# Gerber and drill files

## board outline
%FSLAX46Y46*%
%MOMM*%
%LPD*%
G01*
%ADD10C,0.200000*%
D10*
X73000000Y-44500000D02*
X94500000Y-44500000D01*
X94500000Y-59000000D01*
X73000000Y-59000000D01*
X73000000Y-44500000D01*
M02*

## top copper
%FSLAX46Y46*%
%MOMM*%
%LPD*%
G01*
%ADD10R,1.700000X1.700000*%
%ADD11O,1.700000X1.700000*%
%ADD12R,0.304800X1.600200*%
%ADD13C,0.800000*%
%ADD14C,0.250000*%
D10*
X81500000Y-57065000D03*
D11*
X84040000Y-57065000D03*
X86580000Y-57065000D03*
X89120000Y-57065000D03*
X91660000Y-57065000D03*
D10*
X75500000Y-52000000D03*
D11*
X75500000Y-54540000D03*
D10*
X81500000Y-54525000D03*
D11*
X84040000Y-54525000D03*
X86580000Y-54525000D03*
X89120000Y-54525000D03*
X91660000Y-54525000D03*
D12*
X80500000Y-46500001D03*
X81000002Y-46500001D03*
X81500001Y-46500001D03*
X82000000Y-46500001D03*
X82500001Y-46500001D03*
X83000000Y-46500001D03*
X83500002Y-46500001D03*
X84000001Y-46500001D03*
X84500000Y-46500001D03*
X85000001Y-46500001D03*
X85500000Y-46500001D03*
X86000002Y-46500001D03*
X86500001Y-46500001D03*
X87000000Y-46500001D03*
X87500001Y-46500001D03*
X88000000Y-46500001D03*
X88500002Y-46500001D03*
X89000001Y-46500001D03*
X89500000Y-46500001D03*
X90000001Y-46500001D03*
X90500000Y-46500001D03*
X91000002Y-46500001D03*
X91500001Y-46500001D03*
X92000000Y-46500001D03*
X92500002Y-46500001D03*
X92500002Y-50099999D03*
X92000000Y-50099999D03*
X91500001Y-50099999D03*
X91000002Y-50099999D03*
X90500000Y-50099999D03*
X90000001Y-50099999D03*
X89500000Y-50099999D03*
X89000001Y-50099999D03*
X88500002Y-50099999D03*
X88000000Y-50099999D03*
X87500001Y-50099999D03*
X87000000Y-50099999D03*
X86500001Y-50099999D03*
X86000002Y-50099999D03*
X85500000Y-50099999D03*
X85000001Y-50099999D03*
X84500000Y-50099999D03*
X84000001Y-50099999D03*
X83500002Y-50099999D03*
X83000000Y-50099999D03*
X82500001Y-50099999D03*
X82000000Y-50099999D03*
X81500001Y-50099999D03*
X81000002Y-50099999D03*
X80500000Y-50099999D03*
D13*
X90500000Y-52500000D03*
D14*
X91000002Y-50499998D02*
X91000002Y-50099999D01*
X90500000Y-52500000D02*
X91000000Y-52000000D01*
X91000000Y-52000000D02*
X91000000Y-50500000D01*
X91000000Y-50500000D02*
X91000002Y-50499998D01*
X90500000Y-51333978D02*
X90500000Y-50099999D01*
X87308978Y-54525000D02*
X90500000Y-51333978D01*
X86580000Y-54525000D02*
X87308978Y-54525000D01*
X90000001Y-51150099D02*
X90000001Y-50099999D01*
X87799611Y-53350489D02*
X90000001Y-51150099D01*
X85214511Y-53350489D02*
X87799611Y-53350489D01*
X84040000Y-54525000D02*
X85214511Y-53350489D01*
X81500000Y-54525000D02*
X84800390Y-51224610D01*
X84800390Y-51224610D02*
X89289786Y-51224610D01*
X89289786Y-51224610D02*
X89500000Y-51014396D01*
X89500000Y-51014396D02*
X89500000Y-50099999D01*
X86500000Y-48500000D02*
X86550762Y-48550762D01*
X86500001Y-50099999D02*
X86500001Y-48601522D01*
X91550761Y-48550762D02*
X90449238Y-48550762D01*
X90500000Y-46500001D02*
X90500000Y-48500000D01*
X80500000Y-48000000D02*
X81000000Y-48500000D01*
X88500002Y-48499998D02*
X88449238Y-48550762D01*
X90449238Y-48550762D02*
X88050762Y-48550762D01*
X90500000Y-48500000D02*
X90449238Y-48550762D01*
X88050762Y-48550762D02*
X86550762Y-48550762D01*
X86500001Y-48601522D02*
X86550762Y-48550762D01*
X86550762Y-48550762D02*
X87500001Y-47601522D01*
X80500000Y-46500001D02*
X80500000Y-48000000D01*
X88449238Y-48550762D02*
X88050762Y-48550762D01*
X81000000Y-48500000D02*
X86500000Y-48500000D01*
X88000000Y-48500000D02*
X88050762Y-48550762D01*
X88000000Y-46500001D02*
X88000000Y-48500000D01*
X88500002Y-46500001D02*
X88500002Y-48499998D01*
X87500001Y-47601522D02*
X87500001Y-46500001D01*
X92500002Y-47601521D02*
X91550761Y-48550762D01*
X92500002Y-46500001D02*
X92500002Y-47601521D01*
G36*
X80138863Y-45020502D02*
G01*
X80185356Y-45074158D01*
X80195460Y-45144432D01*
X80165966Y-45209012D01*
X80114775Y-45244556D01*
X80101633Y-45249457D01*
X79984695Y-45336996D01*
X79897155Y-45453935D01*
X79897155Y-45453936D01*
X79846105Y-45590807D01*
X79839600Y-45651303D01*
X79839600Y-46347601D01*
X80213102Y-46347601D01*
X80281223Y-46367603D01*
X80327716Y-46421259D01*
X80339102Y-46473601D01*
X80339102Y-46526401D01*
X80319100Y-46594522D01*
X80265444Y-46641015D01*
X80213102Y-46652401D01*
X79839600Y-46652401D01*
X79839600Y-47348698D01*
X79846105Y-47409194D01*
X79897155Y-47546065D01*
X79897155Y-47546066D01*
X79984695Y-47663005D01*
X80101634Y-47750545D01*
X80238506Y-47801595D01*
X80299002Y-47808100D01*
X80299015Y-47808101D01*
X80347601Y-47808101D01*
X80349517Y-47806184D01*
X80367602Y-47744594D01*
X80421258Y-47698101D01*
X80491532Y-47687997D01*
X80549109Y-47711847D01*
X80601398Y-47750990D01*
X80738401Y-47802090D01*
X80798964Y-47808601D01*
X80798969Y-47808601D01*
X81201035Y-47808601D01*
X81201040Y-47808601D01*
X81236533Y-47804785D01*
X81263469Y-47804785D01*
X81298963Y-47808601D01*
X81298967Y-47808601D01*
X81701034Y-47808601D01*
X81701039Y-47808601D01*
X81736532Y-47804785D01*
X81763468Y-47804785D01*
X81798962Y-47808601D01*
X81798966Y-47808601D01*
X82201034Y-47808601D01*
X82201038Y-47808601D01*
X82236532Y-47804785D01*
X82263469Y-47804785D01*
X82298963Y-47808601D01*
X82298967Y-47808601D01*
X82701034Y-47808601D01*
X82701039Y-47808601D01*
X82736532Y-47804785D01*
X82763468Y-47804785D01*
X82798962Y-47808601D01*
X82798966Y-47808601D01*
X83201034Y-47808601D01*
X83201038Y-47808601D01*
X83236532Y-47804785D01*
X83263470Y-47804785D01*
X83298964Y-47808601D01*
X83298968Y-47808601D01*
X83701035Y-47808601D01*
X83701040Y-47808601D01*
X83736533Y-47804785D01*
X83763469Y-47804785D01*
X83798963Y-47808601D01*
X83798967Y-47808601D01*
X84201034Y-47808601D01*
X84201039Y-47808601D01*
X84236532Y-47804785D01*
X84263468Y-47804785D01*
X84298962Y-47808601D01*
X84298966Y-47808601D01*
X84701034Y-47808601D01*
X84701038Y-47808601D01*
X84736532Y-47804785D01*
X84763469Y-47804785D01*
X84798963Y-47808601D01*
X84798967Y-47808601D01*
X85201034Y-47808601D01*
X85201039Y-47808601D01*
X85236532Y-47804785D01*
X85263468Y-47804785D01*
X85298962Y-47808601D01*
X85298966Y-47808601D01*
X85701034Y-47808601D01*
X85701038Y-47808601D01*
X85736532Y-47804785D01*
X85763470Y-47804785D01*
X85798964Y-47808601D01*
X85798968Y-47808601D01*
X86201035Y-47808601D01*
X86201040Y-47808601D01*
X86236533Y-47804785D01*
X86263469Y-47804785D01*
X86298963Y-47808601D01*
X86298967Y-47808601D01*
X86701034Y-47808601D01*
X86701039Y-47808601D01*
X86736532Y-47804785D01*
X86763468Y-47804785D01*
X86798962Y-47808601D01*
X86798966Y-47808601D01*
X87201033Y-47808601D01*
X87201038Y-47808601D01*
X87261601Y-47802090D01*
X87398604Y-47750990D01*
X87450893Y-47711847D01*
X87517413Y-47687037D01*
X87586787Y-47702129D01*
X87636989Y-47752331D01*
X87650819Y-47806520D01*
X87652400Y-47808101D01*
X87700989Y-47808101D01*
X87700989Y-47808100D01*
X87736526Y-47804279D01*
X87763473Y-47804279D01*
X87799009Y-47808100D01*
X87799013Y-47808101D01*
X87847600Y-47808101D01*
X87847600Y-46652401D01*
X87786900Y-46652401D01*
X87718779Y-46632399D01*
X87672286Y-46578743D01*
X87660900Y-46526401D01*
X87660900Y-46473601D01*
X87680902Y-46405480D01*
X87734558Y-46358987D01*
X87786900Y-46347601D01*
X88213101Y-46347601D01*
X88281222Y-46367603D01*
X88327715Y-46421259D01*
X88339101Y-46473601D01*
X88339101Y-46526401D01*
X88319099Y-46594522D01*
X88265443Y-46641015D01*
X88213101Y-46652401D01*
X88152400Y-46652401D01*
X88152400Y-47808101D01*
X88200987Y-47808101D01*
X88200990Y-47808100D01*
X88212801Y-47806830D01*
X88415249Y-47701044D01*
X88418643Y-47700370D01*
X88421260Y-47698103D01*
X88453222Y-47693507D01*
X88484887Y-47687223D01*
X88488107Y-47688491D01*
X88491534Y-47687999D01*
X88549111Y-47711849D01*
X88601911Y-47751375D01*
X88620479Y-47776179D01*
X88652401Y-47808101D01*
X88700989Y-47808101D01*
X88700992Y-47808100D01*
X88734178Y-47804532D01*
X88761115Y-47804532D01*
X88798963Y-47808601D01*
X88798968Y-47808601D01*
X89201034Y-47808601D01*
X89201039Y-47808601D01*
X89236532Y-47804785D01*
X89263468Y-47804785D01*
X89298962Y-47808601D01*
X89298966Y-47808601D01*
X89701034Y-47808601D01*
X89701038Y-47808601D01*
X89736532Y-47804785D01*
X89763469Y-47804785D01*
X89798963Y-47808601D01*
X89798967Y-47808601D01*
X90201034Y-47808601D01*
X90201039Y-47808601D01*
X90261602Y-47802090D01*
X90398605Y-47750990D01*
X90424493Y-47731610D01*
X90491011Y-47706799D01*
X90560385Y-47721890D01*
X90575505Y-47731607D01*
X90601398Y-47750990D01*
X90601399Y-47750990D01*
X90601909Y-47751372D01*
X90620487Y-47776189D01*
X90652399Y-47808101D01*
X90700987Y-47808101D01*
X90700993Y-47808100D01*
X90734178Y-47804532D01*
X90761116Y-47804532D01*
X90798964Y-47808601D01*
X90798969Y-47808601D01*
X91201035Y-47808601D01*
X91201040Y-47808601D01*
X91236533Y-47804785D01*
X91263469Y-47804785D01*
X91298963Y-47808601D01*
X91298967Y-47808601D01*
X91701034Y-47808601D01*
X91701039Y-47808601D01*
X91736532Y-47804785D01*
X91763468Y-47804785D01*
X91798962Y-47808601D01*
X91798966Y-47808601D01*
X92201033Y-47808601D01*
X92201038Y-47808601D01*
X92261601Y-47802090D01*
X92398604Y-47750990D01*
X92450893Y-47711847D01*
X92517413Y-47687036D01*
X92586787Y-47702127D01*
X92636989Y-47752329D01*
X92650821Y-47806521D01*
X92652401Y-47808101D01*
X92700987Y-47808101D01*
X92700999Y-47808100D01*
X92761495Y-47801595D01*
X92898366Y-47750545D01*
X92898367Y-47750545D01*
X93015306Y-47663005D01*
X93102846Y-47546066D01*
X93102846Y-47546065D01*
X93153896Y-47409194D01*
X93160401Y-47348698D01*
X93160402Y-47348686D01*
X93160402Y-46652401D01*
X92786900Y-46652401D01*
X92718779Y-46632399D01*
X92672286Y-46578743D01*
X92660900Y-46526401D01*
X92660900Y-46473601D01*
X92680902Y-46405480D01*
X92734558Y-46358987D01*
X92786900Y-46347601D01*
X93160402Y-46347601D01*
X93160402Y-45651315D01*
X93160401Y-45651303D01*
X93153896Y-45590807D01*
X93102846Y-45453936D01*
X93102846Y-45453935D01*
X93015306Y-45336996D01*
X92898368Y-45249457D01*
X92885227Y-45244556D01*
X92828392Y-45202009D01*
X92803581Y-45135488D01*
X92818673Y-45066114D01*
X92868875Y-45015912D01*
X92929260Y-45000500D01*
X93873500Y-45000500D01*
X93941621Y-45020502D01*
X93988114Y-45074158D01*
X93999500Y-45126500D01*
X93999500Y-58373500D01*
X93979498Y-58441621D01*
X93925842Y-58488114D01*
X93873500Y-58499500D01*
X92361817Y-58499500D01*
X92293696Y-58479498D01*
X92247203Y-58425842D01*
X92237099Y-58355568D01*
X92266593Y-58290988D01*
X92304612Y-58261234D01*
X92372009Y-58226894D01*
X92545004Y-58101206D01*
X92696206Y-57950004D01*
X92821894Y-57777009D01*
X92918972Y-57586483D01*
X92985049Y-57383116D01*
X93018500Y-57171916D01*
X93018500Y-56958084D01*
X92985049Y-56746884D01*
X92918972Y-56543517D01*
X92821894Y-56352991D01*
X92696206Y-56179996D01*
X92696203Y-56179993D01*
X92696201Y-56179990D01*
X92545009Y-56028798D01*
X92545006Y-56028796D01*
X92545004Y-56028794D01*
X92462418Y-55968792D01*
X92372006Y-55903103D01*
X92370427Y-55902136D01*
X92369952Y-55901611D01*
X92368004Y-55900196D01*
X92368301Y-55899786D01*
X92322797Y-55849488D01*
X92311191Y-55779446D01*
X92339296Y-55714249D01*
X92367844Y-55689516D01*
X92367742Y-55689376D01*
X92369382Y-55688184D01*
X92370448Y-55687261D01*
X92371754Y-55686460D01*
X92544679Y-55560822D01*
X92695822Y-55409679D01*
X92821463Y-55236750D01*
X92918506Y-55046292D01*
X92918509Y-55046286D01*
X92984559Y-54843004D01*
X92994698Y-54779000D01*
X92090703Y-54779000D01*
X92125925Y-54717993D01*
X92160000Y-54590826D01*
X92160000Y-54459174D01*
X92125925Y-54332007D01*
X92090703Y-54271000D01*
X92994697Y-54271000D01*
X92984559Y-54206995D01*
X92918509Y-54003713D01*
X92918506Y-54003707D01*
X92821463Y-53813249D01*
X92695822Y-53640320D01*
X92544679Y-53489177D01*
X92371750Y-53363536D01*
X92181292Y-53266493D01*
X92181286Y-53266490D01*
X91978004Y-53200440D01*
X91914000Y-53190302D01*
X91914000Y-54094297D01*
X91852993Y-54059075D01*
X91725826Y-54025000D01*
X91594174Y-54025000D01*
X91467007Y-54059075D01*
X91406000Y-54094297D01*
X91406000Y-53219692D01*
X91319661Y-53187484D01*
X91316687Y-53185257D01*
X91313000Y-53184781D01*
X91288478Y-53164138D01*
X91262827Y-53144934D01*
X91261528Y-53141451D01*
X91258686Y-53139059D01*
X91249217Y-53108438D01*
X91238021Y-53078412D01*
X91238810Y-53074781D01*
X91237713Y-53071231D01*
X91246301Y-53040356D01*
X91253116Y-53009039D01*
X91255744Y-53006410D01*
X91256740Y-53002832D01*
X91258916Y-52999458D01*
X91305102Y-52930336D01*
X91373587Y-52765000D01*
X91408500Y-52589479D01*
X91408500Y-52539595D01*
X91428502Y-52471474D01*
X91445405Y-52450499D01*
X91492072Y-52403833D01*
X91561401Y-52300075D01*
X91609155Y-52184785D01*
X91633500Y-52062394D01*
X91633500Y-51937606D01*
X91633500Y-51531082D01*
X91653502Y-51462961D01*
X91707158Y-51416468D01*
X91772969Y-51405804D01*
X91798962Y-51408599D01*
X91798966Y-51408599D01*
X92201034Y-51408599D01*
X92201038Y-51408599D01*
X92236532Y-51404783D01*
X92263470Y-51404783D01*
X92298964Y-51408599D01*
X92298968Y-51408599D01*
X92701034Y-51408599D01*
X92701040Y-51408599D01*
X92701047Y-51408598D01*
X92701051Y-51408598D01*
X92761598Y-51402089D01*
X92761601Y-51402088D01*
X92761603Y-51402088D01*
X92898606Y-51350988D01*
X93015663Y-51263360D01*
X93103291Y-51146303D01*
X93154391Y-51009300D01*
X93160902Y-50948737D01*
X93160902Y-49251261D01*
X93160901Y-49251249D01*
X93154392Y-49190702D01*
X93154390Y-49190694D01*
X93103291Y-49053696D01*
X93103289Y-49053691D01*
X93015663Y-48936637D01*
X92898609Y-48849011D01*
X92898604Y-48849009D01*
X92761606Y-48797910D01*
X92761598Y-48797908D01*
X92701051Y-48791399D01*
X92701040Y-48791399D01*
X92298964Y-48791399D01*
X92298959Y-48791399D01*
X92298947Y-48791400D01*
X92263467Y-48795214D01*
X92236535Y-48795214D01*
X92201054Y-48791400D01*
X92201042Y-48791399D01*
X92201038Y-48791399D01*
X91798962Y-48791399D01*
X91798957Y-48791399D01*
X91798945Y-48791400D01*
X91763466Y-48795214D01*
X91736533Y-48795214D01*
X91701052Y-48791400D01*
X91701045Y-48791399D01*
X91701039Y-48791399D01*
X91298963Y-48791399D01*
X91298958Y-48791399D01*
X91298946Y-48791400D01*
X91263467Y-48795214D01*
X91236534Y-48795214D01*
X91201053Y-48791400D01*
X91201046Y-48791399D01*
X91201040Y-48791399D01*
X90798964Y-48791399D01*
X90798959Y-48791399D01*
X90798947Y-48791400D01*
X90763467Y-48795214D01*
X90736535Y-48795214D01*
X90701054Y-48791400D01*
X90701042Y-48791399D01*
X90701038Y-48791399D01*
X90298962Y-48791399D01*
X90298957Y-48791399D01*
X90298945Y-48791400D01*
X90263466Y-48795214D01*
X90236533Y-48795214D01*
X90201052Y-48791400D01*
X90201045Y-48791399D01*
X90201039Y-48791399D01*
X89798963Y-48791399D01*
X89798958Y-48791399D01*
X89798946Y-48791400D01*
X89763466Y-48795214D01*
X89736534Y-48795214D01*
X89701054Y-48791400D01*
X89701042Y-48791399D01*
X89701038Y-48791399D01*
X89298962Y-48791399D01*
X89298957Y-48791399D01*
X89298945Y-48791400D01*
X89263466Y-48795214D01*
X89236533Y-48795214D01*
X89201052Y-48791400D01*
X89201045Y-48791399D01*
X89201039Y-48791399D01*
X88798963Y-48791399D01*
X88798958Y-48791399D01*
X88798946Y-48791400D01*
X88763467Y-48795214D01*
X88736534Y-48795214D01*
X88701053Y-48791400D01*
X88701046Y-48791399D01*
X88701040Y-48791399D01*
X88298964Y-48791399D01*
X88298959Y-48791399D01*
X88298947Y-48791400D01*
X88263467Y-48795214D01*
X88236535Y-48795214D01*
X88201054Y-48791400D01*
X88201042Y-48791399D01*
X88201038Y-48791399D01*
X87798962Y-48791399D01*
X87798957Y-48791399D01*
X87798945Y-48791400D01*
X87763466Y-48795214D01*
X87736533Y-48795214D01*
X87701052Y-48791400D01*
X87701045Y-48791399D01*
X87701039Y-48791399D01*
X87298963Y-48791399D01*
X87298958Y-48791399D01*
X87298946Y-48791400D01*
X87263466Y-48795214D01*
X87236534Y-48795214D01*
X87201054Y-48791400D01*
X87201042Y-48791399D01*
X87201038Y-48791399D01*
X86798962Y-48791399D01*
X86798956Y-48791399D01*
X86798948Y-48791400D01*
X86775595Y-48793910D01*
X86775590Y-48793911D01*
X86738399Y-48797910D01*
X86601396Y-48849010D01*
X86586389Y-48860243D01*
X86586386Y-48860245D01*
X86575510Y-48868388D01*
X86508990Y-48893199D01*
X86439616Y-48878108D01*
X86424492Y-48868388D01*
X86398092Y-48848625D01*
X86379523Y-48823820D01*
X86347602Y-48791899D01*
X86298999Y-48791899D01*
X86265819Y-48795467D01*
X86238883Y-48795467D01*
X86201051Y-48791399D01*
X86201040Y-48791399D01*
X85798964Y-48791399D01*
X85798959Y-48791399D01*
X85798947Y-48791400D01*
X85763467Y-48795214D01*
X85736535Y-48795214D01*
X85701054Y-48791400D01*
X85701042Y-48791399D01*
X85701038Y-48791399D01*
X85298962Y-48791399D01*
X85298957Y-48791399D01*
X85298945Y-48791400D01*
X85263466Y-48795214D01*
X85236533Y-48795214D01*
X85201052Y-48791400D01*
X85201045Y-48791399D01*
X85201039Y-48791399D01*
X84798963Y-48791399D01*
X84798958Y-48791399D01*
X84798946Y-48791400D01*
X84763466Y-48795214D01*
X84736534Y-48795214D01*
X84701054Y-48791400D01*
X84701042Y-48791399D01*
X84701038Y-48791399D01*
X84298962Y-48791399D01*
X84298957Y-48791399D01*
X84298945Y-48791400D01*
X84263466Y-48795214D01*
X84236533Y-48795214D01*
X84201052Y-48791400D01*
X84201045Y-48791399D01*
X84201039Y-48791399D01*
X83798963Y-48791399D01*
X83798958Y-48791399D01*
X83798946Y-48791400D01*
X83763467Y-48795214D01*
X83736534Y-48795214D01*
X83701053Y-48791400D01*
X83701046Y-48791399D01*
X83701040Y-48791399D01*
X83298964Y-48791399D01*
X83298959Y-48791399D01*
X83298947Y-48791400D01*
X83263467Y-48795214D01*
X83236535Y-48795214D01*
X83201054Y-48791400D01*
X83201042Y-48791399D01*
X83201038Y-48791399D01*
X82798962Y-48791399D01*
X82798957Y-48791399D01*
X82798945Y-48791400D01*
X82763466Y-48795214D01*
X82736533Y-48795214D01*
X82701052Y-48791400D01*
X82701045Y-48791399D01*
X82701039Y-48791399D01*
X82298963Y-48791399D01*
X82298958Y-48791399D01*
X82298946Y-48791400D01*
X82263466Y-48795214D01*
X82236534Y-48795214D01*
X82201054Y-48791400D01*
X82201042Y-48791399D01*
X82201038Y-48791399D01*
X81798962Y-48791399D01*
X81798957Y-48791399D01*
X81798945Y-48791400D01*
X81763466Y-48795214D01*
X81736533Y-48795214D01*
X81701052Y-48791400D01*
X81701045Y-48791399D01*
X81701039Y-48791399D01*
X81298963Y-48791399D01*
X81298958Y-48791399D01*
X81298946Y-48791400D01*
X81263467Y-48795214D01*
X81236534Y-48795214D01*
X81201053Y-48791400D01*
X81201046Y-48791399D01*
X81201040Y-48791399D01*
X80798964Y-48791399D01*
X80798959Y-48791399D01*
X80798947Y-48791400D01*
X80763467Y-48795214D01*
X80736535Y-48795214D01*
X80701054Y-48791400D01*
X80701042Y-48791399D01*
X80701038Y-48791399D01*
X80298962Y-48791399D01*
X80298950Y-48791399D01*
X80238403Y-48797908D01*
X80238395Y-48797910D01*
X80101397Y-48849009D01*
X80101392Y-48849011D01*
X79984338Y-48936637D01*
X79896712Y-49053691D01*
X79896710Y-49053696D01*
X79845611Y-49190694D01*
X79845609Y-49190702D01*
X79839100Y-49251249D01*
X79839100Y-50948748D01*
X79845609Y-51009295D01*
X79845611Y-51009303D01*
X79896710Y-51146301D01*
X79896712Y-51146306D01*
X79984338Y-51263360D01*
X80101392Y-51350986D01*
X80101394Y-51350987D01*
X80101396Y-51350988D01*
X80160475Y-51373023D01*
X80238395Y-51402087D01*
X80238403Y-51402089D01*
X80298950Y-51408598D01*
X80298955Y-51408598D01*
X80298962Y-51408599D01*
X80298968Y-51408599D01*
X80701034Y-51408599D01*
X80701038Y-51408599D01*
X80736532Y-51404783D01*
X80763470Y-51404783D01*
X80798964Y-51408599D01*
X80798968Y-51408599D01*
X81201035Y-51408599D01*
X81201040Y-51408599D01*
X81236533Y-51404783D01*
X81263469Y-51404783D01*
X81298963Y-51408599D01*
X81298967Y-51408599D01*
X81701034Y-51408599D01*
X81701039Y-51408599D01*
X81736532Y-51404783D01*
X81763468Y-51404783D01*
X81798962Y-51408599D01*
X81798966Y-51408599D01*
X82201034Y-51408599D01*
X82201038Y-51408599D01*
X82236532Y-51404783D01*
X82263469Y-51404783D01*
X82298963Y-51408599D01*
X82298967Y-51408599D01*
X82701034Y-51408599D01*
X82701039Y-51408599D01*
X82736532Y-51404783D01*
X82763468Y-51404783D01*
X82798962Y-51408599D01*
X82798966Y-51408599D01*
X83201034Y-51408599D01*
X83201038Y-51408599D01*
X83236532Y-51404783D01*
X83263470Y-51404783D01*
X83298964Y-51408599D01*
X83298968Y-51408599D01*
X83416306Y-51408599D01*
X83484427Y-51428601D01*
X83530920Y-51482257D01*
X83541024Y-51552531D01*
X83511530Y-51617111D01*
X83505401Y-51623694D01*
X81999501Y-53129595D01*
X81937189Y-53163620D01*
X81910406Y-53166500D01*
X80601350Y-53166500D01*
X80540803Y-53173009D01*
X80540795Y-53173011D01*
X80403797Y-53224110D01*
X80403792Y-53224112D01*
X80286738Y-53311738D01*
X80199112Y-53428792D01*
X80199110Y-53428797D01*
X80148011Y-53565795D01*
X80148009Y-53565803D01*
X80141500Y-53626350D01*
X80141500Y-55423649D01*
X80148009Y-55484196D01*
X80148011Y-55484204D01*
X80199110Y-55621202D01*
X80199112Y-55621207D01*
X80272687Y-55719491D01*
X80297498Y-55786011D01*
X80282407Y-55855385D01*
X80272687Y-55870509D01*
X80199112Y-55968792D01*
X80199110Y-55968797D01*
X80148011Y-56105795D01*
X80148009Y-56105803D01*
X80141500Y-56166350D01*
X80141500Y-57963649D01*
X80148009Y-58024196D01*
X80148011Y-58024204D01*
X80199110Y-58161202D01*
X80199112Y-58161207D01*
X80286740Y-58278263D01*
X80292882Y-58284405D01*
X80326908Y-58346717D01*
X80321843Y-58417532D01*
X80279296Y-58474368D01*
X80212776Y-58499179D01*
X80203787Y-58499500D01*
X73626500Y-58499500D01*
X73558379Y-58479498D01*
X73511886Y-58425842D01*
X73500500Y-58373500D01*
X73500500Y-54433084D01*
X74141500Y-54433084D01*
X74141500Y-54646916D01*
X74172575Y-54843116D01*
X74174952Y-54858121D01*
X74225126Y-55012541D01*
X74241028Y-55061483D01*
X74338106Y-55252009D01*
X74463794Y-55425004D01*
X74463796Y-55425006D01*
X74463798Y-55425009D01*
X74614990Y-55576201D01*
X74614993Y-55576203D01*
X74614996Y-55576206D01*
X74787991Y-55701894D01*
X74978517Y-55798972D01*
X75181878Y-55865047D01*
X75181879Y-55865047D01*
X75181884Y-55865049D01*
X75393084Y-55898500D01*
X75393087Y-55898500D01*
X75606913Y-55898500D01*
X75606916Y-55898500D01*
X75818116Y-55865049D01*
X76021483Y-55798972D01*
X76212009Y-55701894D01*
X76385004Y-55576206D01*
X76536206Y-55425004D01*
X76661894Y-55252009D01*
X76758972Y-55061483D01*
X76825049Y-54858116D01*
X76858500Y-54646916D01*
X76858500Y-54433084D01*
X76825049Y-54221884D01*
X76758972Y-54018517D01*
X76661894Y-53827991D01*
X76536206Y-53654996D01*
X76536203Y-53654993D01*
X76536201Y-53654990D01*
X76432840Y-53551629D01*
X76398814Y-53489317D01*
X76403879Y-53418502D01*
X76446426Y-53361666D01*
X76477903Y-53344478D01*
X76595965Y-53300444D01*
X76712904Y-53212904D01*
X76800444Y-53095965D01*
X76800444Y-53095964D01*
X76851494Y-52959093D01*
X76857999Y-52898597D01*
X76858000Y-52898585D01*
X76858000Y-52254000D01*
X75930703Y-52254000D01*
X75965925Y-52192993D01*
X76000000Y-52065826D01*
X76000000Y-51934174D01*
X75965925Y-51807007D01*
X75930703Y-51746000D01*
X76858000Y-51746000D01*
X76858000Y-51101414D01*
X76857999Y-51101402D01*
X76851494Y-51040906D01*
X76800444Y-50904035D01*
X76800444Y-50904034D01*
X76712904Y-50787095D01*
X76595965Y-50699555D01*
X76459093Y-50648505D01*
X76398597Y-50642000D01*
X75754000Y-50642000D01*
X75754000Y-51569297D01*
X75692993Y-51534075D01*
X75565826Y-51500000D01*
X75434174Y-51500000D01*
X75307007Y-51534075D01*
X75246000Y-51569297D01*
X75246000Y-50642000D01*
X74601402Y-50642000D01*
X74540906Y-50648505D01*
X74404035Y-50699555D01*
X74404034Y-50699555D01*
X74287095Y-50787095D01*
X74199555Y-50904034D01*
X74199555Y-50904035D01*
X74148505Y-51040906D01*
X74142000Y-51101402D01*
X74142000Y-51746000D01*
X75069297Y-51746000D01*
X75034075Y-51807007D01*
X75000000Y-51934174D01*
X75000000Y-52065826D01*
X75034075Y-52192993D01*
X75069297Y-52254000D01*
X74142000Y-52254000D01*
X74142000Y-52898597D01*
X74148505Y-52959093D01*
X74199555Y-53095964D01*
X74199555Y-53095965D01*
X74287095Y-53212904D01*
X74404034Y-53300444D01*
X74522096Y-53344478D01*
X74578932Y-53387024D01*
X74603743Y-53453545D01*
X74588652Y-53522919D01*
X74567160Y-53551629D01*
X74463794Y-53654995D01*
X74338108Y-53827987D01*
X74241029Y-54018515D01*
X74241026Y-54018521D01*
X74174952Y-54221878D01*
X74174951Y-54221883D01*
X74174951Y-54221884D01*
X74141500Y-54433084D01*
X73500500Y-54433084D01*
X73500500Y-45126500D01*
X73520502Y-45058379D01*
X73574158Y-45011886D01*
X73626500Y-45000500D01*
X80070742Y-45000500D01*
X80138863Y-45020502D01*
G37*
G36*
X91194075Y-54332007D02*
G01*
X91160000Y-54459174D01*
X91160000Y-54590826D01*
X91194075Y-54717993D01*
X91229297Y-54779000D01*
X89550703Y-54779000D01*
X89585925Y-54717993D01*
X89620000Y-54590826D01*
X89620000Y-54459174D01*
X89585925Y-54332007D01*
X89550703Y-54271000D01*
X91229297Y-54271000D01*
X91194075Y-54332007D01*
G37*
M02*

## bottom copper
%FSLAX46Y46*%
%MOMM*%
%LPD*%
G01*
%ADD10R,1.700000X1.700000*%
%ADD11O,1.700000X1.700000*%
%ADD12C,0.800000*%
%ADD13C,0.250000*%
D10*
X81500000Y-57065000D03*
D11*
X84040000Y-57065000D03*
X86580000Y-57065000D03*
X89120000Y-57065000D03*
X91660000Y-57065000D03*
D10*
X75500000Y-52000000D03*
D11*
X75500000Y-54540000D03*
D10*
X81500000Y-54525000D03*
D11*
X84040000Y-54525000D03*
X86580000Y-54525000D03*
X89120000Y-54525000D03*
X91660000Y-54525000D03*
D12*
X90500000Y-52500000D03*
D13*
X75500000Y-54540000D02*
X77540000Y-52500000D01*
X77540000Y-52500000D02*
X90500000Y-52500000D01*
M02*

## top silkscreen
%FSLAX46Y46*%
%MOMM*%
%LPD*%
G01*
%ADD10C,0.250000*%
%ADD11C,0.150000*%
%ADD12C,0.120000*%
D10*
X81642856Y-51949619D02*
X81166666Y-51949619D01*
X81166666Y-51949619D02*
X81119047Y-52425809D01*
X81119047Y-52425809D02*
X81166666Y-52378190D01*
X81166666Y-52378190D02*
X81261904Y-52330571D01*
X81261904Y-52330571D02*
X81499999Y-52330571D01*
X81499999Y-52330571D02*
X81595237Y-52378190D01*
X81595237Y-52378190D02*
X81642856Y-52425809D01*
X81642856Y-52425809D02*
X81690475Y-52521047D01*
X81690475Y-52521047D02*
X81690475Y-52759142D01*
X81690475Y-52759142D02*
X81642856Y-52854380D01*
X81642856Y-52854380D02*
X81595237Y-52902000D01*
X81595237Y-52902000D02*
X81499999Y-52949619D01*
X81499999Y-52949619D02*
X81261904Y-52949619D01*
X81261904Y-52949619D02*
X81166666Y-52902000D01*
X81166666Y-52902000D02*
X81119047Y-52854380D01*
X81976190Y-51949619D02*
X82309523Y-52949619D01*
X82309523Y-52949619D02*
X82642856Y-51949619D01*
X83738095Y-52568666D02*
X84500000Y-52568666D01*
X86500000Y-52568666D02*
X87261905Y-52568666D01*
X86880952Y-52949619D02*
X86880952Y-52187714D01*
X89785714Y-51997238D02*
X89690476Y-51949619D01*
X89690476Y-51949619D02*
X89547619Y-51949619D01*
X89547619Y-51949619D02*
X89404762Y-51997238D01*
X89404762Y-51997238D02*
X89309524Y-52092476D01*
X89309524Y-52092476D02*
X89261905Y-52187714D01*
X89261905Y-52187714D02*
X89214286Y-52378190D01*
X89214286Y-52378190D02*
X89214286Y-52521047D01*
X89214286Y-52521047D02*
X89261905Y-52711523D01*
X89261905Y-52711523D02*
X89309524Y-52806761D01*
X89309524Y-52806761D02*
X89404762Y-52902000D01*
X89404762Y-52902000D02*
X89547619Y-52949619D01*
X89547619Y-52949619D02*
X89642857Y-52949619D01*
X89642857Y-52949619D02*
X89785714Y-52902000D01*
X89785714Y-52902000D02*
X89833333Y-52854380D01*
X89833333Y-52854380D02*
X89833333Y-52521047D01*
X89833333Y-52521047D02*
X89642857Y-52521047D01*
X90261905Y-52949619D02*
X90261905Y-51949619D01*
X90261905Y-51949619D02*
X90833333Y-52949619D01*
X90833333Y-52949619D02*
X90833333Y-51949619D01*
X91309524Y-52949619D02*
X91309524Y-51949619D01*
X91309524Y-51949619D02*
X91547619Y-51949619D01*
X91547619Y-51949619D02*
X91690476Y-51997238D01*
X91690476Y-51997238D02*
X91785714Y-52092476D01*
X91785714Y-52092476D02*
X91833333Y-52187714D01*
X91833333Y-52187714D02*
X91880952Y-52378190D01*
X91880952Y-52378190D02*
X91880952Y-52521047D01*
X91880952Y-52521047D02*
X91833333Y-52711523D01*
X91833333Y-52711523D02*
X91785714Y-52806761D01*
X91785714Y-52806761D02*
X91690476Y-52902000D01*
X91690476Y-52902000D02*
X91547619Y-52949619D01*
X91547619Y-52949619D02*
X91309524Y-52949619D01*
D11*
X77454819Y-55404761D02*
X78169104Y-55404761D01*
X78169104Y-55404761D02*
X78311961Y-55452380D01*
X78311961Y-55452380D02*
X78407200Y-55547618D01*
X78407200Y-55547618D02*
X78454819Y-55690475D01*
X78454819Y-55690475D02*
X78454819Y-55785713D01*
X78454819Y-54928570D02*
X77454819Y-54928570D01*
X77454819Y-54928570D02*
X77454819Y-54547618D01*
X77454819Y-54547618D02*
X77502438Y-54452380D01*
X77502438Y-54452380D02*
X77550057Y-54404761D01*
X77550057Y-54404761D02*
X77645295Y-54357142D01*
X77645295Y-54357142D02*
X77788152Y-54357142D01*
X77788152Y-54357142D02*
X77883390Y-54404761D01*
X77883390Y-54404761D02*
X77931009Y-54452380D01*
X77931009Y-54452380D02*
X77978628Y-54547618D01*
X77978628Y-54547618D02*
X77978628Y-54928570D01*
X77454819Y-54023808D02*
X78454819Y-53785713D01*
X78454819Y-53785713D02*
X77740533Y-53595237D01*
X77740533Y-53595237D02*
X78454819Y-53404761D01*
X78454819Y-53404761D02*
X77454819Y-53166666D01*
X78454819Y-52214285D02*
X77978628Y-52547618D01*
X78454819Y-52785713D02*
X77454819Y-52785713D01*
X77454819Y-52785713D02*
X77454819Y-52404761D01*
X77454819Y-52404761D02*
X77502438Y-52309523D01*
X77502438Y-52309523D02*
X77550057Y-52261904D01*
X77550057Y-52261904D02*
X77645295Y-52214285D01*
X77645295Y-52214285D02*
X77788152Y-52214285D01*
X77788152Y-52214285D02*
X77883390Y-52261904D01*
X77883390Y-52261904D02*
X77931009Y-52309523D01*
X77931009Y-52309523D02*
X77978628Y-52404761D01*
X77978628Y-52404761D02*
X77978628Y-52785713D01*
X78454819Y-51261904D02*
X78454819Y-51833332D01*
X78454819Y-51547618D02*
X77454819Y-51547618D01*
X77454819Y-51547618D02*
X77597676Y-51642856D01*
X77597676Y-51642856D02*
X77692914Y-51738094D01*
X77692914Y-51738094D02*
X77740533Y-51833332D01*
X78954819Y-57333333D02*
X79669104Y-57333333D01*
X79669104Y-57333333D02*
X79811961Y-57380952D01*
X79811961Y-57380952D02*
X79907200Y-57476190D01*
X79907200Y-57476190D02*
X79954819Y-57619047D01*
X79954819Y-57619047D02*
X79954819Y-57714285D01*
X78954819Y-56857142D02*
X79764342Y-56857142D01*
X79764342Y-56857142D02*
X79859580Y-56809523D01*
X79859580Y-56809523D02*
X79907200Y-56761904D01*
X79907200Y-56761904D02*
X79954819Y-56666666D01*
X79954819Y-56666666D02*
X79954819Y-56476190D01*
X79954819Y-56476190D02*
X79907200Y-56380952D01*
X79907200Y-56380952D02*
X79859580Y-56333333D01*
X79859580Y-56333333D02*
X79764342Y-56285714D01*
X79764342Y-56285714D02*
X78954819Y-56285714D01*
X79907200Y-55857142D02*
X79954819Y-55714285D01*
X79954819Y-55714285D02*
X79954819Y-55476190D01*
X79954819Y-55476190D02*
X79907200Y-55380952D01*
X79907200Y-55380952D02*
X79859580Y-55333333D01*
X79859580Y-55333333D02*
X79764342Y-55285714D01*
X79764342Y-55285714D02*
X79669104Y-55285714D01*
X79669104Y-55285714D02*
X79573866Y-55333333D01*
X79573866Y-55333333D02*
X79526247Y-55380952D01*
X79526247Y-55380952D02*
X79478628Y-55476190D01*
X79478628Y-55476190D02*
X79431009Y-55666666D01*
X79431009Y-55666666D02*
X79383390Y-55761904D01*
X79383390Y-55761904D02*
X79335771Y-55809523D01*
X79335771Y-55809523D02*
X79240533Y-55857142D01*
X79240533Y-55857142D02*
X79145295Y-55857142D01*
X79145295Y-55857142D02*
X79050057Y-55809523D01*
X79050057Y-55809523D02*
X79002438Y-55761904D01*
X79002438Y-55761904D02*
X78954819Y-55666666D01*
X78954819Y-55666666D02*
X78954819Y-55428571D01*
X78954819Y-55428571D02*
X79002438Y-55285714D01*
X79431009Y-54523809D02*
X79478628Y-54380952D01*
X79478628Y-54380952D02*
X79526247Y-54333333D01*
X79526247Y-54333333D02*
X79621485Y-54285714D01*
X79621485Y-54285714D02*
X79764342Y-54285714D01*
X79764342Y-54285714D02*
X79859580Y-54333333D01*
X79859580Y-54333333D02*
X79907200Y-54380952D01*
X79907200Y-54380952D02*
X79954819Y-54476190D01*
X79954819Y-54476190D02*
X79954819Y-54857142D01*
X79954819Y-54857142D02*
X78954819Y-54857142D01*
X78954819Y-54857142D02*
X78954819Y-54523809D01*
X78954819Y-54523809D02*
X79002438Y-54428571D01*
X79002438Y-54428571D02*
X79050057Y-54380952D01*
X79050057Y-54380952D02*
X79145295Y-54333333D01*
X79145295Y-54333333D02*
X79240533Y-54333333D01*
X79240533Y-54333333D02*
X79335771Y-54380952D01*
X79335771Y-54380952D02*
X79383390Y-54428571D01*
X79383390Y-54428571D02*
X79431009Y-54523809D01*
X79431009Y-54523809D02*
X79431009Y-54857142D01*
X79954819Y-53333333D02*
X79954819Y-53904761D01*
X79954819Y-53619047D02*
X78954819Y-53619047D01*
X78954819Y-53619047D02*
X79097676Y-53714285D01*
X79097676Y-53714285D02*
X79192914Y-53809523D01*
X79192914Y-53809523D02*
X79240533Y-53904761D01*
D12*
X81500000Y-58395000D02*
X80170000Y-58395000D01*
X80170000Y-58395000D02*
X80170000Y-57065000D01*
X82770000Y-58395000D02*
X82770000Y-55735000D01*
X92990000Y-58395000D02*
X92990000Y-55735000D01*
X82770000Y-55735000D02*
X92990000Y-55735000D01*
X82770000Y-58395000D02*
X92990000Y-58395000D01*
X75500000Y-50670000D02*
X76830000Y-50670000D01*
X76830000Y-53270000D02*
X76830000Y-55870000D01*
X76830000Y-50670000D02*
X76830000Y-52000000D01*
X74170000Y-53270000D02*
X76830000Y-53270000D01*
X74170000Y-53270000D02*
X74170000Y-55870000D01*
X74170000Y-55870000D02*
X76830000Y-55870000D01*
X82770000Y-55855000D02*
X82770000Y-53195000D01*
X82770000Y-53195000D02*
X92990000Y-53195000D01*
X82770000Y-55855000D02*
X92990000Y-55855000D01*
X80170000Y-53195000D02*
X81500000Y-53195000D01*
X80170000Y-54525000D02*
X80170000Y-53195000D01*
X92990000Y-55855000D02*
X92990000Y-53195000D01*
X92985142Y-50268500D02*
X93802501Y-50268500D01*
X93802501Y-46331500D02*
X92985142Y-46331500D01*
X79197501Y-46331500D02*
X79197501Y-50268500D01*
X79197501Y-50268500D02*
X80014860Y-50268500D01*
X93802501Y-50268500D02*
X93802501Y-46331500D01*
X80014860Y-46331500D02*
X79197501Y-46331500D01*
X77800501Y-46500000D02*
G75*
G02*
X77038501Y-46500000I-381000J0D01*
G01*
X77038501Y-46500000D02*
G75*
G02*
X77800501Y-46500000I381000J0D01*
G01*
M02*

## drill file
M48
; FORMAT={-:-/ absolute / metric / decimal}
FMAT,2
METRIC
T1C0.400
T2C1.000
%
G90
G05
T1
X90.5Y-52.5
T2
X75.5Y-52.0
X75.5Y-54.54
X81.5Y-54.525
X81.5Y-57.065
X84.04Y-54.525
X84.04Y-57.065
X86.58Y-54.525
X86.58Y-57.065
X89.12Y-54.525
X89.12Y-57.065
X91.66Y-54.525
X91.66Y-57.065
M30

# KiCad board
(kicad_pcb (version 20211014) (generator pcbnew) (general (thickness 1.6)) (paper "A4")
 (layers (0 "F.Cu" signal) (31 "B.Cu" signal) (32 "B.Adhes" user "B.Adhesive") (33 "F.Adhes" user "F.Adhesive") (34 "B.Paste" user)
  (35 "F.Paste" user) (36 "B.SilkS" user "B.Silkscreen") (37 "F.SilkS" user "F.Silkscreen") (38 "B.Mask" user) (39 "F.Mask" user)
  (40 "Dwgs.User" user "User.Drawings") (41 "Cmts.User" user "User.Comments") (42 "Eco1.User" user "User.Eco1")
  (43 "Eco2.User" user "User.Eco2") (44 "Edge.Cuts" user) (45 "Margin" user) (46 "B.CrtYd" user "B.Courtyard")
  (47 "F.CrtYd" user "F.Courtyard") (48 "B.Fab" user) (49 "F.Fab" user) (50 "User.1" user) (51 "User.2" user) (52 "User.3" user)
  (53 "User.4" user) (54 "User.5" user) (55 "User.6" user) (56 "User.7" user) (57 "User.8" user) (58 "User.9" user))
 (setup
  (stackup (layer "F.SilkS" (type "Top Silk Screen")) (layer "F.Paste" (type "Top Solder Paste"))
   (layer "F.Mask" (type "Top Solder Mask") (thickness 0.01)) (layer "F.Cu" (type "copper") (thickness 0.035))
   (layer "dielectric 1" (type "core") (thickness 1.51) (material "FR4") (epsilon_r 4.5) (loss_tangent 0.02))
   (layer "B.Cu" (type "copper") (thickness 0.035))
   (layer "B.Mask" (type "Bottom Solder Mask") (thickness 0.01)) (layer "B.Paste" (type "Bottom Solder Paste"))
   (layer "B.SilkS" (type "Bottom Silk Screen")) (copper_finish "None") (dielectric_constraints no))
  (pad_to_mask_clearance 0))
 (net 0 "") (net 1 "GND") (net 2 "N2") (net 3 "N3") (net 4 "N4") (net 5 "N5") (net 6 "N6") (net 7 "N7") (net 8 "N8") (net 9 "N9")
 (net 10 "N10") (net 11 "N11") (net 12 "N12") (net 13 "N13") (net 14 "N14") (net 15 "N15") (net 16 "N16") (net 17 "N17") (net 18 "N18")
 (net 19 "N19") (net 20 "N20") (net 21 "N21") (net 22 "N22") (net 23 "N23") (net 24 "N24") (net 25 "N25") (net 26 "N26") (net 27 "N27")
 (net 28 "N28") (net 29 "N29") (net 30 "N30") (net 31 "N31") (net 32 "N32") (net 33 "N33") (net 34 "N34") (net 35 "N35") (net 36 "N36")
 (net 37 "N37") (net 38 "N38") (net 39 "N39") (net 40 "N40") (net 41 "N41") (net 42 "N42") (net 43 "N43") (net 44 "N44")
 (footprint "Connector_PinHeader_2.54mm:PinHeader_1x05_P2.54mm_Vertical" (layer "F.Cu") (at 81.5 57.065 90)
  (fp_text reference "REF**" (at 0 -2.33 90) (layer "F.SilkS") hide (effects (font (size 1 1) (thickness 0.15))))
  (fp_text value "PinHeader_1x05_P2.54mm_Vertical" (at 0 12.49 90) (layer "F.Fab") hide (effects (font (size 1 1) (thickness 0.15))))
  (fp_line (start -1.33 0) (end -1.33 -1.33) (layer "F.SilkS") (width 0.12))
  (fp_line (start -1.33 -1.33) (end 0 -1.33) (layer "F.SilkS") (width 0.12))
  (fp_line (start -1.33 1.27) (end 1.33 1.27) (layer "F.SilkS") (width 0.12))
  (fp_line (start -1.33 11.49) (end 1.33 11.49) (layer "F.SilkS") (width 0.12))
  (fp_line (start 1.33 1.27) (end 1.33 11.49) (layer "F.SilkS") (width 0.12))
  (fp_line (start -1.33 1.27) (end -1.33 11.49) (layer "F.SilkS") (width 0.12))
  (pad "1" thru_hole rect (at 0 0 90) (size 1.7 1.7) (drill 1) (layers *.Cu *.Mask))
  (pad "2" thru_hole oval (at 0 2.54 90) (size 1.7 1.7) (drill 1) (layers *.Cu *.Mask))
  (pad "3" thru_hole oval (at 0 5.08 90) (size 1.7 1.7) (drill 1) (layers *.Cu *.Mask))
  (pad "4" thru_hole oval (at 0 7.62 90) (size 1.7 1.7) (drill 1) (layers *.Cu *.Mask))
  (pad "5" thru_hole oval (at 0 10.16 90) (size 1.7 1.7) (drill 1) (layers *.Cu *.Mask)))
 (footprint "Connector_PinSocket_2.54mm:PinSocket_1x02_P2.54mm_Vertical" (layer "F.Cu") (at 75.5 52)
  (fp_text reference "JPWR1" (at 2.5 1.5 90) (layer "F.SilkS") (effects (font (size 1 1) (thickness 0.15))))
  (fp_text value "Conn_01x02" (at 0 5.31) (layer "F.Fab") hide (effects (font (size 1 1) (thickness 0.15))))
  (fp_line (start 0 -1.33) (end 1.33 -1.33) (layer "F.SilkS") (width 0.12))
  (fp_line (start 1.33 1.27) (end 1.33 3.87) (layer "F.SilkS") (width 0.12))
  (fp_line (start 1.33 -1.33) (end 1.33 0) (layer "F.SilkS") (width 0.12))
  (fp_line (start -1.33 1.27) (end 1.33 1.27) (layer "F.SilkS") (width 0.12))
  (fp_line (start -1.33 1.27) (end -1.33 3.87) (layer "F.SilkS") (width 0.12))
  (fp_line (start -1.33 3.87) (end 1.33 3.87) (layer "F.SilkS") (width 0.12))
  (pad "1" thru_hole rect (at 0 0) (size 1.7 1.7) (drill 1) (layers *.Cu *.Mask) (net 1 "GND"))
  (pad "2" thru_hole oval (at 0 2.54) (size 1.7 1.7) (drill 1) (layers *.Cu *.Mask) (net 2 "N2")))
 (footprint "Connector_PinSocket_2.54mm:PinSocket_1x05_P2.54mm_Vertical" (layer "F.Cu") (at 81.5 54.525 90)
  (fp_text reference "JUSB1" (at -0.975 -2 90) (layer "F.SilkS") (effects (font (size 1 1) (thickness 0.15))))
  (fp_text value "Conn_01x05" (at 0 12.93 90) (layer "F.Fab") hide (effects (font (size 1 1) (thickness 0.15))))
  (fp_line (start -1.33 1.27) (end 1.33 1.27) (layer "F.SilkS") (width 0.12))
  (fp_line (start 1.33 1.27) (end 1.33 11.49) (layer "F.SilkS") (width 0.12))
  (fp_line (start -1.33 1.27) (end -1.33 11.49) (layer "F.SilkS") (width 0.12))
  (fp_line (start 1.33 -1.33) (end 1.33 0) (layer "F.SilkS") (width 0.12))
  (fp_line (start 0 -1.33) (end 1.33 -1.33) (layer "F.SilkS") (width 0.12))
  (fp_line (start -1.33 11.49) (end 1.33 11.49) (layer "F.SilkS") (width 0.12))
  (pad "1" thru_hole rect (at 0 0 90) (size 1.7 1.7) (drill 1) (layers *.Cu *.Mask) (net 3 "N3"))
  (pad "2" thru_hole oval (at 0 2.54 90) (size 1.7 1.7) (drill 1) (layers *.Cu *.Mask) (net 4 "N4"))
  (pad "3" thru_hole oval (at 0 5.08 90) (size 1.7 1.7) (drill 1) (layers *.Cu *.Mask) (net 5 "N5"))
  (pad "4" thru_hole oval (at 0 7.62 90) (size 1.7 1.7) (drill 1) (layers *.Cu *.Mask) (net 1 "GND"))
  (pad "5" thru_hole oval (at 0 10.16 90) (size 1.7 1.7) (drill 1) (layers *.Cu *.Mask) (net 1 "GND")))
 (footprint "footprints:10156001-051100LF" (layer "F.Cu") (at 80.5 46.5)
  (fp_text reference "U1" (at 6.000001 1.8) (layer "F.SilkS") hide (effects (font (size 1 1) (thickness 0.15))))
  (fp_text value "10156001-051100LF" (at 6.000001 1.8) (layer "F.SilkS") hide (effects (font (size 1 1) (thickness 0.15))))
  (fp_line (start 12.485142 3.7685) (end 13.302501 3.7685) (layer "F.SilkS") (width 0.12))
  (fp_line (start 13.302501 -0.1685) (end 12.485142 -0.1685) (layer "F.SilkS") (width 0.12))
  (fp_line (start -1.302499 -0.1685) (end -1.302499 3.7685) (layer "F.SilkS") (width 0.12))
  (fp_line (start -1.302499 3.7685) (end -0.48514 3.7685) (layer "F.SilkS") (width 0.12))
  (fp_line (start 13.302501 3.7685) (end 13.302501 -0.1685) (layer "F.SilkS") (width 0.12))
  (fp_line (start -0.48514 -0.1685) (end -1.302499 -0.1685) (layer "F.SilkS") (width 0.12))
  (fp_circle (center -3.080499 0) (end -2.699499 0) (layer "F.SilkS") (width 0.12) (fill none))
  (pad "1" smd rect locked (at 0 0.000001) (size 0.3048 1.6002) (layers "F.Cu" "F.Paste" "F.Mask") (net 1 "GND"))
  (pad "2" smd rect locked (at 0.500002 0.000001) (size 0.3048 1.6002) (layers "F.Cu" "F.Paste" "F.Mask") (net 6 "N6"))
  (pad "3" smd rect locked (at 1.000001 0.000001) (size 0.3048 1.6002) (layers "F.Cu" "F.Paste" "F.Mask") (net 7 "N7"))
  (pad "4" smd rect locked (at 1.5 0.000001) (size 0.3048 1.6002) (layers "F.Cu" "F.Paste" "F.Mask") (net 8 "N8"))
  (pad "5" smd rect locked (at 2.000001 0.000001) (size 0.3048 1.6002) (layers "F.Cu" "F.Paste" "F.Mask") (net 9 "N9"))
  (pad "6" smd rect locked (at 2.5 0.000001) (size 0.3048 1.6002) (layers "F.Cu" "F.Paste" "F.Mask") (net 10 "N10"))
  (pad "7" smd rect locked (at 3.000002 0.000001) (size 0.3048 1.6002) (layers "F.Cu" "F.Paste" "F.Mask") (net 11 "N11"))
  (pad "8" smd rect locked (at 3.500001 0.000001) (size 0.3048 1.6002) (layers "F.Cu" "F.Paste" "F.Mask") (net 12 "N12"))
  (pad "9" smd rect locked (at 4 0.000001) (size 0.3048 1.6002) (layers "F.Cu" "F.Paste" "F.Mask") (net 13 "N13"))
  (pad "10" smd rect locked (at 4.500001 0.000001) (size 0.3048 1.6002) (layers "F.Cu" "F.Paste" "F.Mask") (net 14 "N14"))
  (pad "11" smd rect locked (at 5 0.000001) (size 0.3048 1.6002) (layers "F.Cu" "F.Paste" "F.Mask") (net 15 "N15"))
  (pad "12" smd rect locked (at 5.500002 0.000001) (size 0.3048 1.6002) (layers "F.Cu" "F.Paste" "F.Mask") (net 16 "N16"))
  (pad "13" smd rect locked (at 6.000001 0.000001) (size 0.3048 1.6002) (layers "F.Cu" "F.Paste" "F.Mask") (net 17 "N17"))
  (pad "14" smd rect locked (at 6.5 0.000001) (size 0.3048 1.6002) (layers "F.Cu" "F.Paste" "F.Mask") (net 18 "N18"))
  (pad "15" smd rect locked (at 7.000001 0.000001) (size 0.3048 1.6002) (layers "F.Cu" "F.Paste" "F.Mask") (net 1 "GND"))
  (pad "16" smd rect locked (at 7.5 0.000001) (size 0.3048 1.6002) (layers "F.Cu" "F.Paste" "F.Mask") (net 1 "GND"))
  (pad "17" smd rect locked (at 8.000002 0.000001) (size 0.3048 1.6002) (layers "F.Cu" "F.Paste" "F.Mask") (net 1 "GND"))
  (pad "18" smd rect locked (at 8.500001 0.000001) (size 0.3048 1.6002) (layers "F.Cu" "F.Paste" "F.Mask") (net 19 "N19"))
  (pad "19" smd rect locked (at 9 0.000001) (size 0.3048 1.6002) (layers "F.Cu" "F.Paste" "F.Mask") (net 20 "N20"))
  (pad "20" smd rect locked (at 9.500001 0.000001) (size 0.3048 1.6002) (layers "F.Cu" "F.Paste" "F.Mask") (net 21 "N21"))
  (pad "21" smd rect locked (at 10 0.000001) (size 0.3048 1.6002) (layers "F.Cu" "F.Paste" "F.Mask") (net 1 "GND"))
  (pad "22" smd rect locked (at 10.500002 0.000001) (size 0.3048 1.6002) (layers "F.Cu" "F.Paste" "F.Mask") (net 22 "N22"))
  (pad "23" smd rect locked (at 11.000001 0.000001) (size 0.3048 1.6002) (layers "F.Cu" "F.Paste" "F.Mask") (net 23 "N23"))
  (pad "24" smd rect locked (at 11.5 0.000001) (size 0.3048 1.6002) (layers "F.Cu" "F.Paste" "F.Mask") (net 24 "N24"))
  (pad "25" smd rect locked (at 12.000002 0.000001) (size 0.3048 1.6002) (layers "F.Cu" "F.Paste" "F.Mask") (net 1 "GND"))
  (pad "26" smd rect locked (at 12.000002 3.599999) (size 0.3048 1.6002) (layers "F.Cu" "F.Paste" "F.Mask") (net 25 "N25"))
  (pad "27" smd rect locked (at 11.5 3.599999) (size 0.3048 1.6002) (layers "F.Cu" "F.Paste" "F.Mask") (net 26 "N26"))
  (pad "28" smd rect locked (at 11.000001 3.599999) (size 0.3048 1.6002) (layers "F.Cu" "F.Paste" "F.Mask") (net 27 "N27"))
  (pad "29" smd rect locked (at 10.500002 3.599999) (size 0.3048 1.6002) (layers "F.Cu" "F.Paste" "F.Mask") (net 2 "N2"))
  (pad "30" smd rect locked (at 10 3.599999) (size 0.3048 1.6002) (layers "F.Cu" "F.Paste" "F.Mask") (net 5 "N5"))
  (pad "31" smd rect locked (at 9.500001 3.599999) (size 0.3048 1.6002) (layers "F.Cu" "F.Paste" "F.Mask") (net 4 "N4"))
  (pad "32" smd rect locked (at 9 3.599999) (size 0.3048 1.6002) (layers "F.Cu" "F.Paste" "F.Mask") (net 3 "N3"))
  (pad "33" smd rect locked (at 8.500001 3.599999) (size 0.3048 1.6002) (layers "F.Cu" "F.Paste" "F.Mask") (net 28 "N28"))
  (pad "34" smd rect locked (at 8.000002 3.599999) (size 0.3048 1.6002) (layers "F.Cu" "F.Paste" "F.Mask") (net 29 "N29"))
  (pad "35" smd rect locked (at 7.5 3.599999) (size 0.3048 1.6002) (layers "F.Cu" "F.Paste" "F.Mask") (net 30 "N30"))
  (pad "36" smd rect locked (at 7.000001 3.599999) (size 0.3048 1.6002) (layers "F.Cu" "F.Paste" "F.Mask") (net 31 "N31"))
  (pad "37" smd rect locked (at 6.5 3.599999) (size 0.3048 1.6002) (layers "F.Cu" "F.Paste" "F.Mask") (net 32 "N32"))
  (pad "38" smd rect locked (at 6.000001 3.599999) (size 0.3048 1.6002) (layers "F.Cu" "F.Paste" "F.Mask") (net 1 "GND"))
  (pad "39" smd rect locked (at 5.500002 3.599999) (size 0.3048 1.6002) (layers "F.Cu" "F.Paste" "F.Mask") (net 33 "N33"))
  (pad "40" smd rect locked (at 5 3.599999) (size 0.3048 1.6002) (layers "F.Cu" "F.Paste" "F.Mask") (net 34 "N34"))
  (pad "41" smd rect locked (at 4.500001 3.599999) (size 0.3048 1.6002) (layers "F.Cu" "F.Paste" "F.Mask") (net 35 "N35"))
  (pad "42" smd rect locked (at 4 3.599999) (size 0.3048 1.6002) (layers "F.Cu" "F.Paste" "F.Mask") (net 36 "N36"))
  (pad "43" smd rect locked (at 3.500001 3.599999) (size 0.3048 1.6002) (layers "F.Cu" "F.Paste" "F.Mask") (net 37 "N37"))
  (pad "44" smd rect locked (at 3.000002 3.599999) (size 0.3048 1.6002) (layers "F.Cu" "F.Paste" "F.Mask") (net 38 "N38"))
  (pad "45" smd rect locked (at 2.5 3.599999) (size 0.3048 1.6002) (layers "F.Cu" "F.Paste" "F.Mask") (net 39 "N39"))
  (pad "46" smd rect locked (at 2.000001 3.599999) (size 0.3048 1.6002) (layers "F.Cu" "F.Paste" "F.Mask") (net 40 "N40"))
  (pad "47" smd rect locked (at 1.5 3.599999) (size 0.3048 1.6002) (layers "F.Cu" "F.Paste" "F.Mask") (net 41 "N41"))
  (pad "48" smd rect locked (at 1.000001 3.599999) (size 0.3048 1.6002) (layers "F.Cu" "F.Paste" "F.Mask") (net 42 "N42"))
  (pad "49" smd rect locked (at 0.500002 3.599999) (size 0.3048 1.6002) (layers "F.Cu" "F.Paste" "F.Mask") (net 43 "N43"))
  (pad "50" smd rect locked (at 0 3.599999) (size 0.3048 1.6002) (layers "F.Cu" "F.Paste" "F.Mask") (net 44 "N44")))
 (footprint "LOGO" (layer "B.Cu") (at 85.5 49 180)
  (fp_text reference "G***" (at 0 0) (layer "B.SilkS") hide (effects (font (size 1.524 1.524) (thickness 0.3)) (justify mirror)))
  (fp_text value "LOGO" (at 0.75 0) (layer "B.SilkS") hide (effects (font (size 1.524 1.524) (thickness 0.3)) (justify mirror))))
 (gr_rect (start 94.5 59) (end 73 44.5) (layer "Edge.Cuts") (width 0.2) (fill none))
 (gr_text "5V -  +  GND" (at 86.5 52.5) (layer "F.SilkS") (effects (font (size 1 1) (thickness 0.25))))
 (segment (start 91.000002 50.499998) (end 91.000002 50.099999) (width 0.25) (layer "F.Cu") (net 2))
 (segment (start 90.5 52.5) (end 91 52) (width 0.25) (layer "F.Cu") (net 2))
 (segment (start 91 52) (end 91 50.5) (width 0.25) (layer "F.Cu") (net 2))
 (segment (start 91 50.5) (end 91.000002 50.499998) (width 0.25) (layer "F.Cu") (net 2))
 (via (at 90.5 52.5) (size 0.8) (drill 0.4) (layers "F.Cu" "B.Cu") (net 2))
 (segment (start 75.5 54.54) (end 77.54 52.5) (width 0.25) (layer "B.Cu") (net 2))
 (segment (start 77.54 52.5) (end 90.5 52.5) (width 0.25) (layer "B.Cu") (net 2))
 (segment (start 90.5 51.333978) (end 90.5 50.099999) (width 0.25) (layer "F.Cu") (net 5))
 (segment (start 87.308978 54.525) (end 90.5 51.333978) (width 0.25) (layer "F.Cu") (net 5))
 (segment (start 86.58 54.525) (end 87.308978 54.525) (width 0.25) (layer "F.Cu") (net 5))
 (segment (start 90.000001 51.150099) (end 90.000001 50.099999) (width 0.25) (layer "F.Cu") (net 4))
 (segment (start 87.799611 53.350489) (end 90.000001 51.150099) (width 0.25) (layer "F.Cu") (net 4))
 (segment (start 85.214511 53.350489) (end 87.799611 53.350489) (width 0.25) (layer "F.Cu") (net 4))
 (segment (start 84.04 54.525) (end 85.214511 53.350489) (width 0.25) (layer "F.Cu") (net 4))
 (segment (start 81.5 54.525) (end 84.80039 51.22461) (width 0.25) (layer "F.Cu") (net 3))
 (segment (start 84.80039 51.22461) (end 89.289786 51.22461) (width 0.25) (layer "F.Cu") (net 3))
 (segment (start 89.289786 51.22461) (end 89.5 51.014396) (width 0.25) (layer "F.Cu") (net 3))
 (segment (start 89.5 51.014396) (end 89.5 50.099999) (width 0.25) (layer "F.Cu") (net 3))
 (segment (start 86.5 48.5) (end 86.550762 48.550762) (width 0.25) (layer "F.Cu") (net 1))
 (segment (start 86.500001 50.099999) (end 86.500001 48.601522) (width 0.25) (layer "F.Cu") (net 1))
 (segment (start 91.550761 48.550762) (end 90.449238 48.550762) (width 0.25) (layer "F.Cu") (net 1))
 (segment (start 90.5 46.500001) (end 90.5 48.5) (width 0.25) (layer "F.Cu") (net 1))
 (segment (start 80.5 48) (end 81 48.5) (width 0.25) (layer "F.Cu") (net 1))
 (segment (start 88.500002 48.499998) (end 88.449238 48.550762) (width 0.25) (layer "F.Cu") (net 1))
 (segment (start 90.449238 48.550762) (end 88.050762 48.550762) (width 0.25) (layer "F.Cu") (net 1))
 (segment (start 90.5 48.5) (end 90.449238 48.550762) (width 0.25) (layer "F.Cu") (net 1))
 (segment (start 88.050762 48.550762) (end 86.550762 48.550762) (width 0.25) (layer "F.Cu") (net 1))
 (segment (start 86.500001 48.601522) (end 86.550762 48.550762) (width 0.25) (layer "F.Cu") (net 1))
 (segment (start 86.550762 48.550762) (end 87.500001 47.601522) (width 0.25) (layer "F.Cu") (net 1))
 (segment (start 80.5 46.500001) (end 80.5 48) (width 0.25) (layer "F.Cu") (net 1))
 (segment (start 88.449238 48.550762) (end 88.050762 48.550762) (width 0.25) (layer "F.Cu") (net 1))
 (segment (start 81 48.5) (end 86.5 48.5) (width 0.25) (layer "F.Cu") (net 1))
 (segment (start 88 48.5) (end 88.050762 48.550762) (width 0.25) (layer "F.Cu") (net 1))
 (segment (start 88 46.500001) (end 88 48.5) (width 0.25) (layer "F.Cu") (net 1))
 (segment (start 88.500002 46.500001) (end 88.500002 48.499998) (width 0.25) (layer "F.Cu") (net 1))
 (segment (start 87.500001 47.601522) (end 87.500001 46.500001) (width 0.25) (layer "F.Cu") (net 1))
 (segment (start 92.500002 47.601521) (end 91.550761 48.550762) (width 0.25) (layer "F.Cu") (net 1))
 (segment (start 92.500002 46.500001) (end 92.500002 47.601521) (width 0.25) (layer "F.Cu") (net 1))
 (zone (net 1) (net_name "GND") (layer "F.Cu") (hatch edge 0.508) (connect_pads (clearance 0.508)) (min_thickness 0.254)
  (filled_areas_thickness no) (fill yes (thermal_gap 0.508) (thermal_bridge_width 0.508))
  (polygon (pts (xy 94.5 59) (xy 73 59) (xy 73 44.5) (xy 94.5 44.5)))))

